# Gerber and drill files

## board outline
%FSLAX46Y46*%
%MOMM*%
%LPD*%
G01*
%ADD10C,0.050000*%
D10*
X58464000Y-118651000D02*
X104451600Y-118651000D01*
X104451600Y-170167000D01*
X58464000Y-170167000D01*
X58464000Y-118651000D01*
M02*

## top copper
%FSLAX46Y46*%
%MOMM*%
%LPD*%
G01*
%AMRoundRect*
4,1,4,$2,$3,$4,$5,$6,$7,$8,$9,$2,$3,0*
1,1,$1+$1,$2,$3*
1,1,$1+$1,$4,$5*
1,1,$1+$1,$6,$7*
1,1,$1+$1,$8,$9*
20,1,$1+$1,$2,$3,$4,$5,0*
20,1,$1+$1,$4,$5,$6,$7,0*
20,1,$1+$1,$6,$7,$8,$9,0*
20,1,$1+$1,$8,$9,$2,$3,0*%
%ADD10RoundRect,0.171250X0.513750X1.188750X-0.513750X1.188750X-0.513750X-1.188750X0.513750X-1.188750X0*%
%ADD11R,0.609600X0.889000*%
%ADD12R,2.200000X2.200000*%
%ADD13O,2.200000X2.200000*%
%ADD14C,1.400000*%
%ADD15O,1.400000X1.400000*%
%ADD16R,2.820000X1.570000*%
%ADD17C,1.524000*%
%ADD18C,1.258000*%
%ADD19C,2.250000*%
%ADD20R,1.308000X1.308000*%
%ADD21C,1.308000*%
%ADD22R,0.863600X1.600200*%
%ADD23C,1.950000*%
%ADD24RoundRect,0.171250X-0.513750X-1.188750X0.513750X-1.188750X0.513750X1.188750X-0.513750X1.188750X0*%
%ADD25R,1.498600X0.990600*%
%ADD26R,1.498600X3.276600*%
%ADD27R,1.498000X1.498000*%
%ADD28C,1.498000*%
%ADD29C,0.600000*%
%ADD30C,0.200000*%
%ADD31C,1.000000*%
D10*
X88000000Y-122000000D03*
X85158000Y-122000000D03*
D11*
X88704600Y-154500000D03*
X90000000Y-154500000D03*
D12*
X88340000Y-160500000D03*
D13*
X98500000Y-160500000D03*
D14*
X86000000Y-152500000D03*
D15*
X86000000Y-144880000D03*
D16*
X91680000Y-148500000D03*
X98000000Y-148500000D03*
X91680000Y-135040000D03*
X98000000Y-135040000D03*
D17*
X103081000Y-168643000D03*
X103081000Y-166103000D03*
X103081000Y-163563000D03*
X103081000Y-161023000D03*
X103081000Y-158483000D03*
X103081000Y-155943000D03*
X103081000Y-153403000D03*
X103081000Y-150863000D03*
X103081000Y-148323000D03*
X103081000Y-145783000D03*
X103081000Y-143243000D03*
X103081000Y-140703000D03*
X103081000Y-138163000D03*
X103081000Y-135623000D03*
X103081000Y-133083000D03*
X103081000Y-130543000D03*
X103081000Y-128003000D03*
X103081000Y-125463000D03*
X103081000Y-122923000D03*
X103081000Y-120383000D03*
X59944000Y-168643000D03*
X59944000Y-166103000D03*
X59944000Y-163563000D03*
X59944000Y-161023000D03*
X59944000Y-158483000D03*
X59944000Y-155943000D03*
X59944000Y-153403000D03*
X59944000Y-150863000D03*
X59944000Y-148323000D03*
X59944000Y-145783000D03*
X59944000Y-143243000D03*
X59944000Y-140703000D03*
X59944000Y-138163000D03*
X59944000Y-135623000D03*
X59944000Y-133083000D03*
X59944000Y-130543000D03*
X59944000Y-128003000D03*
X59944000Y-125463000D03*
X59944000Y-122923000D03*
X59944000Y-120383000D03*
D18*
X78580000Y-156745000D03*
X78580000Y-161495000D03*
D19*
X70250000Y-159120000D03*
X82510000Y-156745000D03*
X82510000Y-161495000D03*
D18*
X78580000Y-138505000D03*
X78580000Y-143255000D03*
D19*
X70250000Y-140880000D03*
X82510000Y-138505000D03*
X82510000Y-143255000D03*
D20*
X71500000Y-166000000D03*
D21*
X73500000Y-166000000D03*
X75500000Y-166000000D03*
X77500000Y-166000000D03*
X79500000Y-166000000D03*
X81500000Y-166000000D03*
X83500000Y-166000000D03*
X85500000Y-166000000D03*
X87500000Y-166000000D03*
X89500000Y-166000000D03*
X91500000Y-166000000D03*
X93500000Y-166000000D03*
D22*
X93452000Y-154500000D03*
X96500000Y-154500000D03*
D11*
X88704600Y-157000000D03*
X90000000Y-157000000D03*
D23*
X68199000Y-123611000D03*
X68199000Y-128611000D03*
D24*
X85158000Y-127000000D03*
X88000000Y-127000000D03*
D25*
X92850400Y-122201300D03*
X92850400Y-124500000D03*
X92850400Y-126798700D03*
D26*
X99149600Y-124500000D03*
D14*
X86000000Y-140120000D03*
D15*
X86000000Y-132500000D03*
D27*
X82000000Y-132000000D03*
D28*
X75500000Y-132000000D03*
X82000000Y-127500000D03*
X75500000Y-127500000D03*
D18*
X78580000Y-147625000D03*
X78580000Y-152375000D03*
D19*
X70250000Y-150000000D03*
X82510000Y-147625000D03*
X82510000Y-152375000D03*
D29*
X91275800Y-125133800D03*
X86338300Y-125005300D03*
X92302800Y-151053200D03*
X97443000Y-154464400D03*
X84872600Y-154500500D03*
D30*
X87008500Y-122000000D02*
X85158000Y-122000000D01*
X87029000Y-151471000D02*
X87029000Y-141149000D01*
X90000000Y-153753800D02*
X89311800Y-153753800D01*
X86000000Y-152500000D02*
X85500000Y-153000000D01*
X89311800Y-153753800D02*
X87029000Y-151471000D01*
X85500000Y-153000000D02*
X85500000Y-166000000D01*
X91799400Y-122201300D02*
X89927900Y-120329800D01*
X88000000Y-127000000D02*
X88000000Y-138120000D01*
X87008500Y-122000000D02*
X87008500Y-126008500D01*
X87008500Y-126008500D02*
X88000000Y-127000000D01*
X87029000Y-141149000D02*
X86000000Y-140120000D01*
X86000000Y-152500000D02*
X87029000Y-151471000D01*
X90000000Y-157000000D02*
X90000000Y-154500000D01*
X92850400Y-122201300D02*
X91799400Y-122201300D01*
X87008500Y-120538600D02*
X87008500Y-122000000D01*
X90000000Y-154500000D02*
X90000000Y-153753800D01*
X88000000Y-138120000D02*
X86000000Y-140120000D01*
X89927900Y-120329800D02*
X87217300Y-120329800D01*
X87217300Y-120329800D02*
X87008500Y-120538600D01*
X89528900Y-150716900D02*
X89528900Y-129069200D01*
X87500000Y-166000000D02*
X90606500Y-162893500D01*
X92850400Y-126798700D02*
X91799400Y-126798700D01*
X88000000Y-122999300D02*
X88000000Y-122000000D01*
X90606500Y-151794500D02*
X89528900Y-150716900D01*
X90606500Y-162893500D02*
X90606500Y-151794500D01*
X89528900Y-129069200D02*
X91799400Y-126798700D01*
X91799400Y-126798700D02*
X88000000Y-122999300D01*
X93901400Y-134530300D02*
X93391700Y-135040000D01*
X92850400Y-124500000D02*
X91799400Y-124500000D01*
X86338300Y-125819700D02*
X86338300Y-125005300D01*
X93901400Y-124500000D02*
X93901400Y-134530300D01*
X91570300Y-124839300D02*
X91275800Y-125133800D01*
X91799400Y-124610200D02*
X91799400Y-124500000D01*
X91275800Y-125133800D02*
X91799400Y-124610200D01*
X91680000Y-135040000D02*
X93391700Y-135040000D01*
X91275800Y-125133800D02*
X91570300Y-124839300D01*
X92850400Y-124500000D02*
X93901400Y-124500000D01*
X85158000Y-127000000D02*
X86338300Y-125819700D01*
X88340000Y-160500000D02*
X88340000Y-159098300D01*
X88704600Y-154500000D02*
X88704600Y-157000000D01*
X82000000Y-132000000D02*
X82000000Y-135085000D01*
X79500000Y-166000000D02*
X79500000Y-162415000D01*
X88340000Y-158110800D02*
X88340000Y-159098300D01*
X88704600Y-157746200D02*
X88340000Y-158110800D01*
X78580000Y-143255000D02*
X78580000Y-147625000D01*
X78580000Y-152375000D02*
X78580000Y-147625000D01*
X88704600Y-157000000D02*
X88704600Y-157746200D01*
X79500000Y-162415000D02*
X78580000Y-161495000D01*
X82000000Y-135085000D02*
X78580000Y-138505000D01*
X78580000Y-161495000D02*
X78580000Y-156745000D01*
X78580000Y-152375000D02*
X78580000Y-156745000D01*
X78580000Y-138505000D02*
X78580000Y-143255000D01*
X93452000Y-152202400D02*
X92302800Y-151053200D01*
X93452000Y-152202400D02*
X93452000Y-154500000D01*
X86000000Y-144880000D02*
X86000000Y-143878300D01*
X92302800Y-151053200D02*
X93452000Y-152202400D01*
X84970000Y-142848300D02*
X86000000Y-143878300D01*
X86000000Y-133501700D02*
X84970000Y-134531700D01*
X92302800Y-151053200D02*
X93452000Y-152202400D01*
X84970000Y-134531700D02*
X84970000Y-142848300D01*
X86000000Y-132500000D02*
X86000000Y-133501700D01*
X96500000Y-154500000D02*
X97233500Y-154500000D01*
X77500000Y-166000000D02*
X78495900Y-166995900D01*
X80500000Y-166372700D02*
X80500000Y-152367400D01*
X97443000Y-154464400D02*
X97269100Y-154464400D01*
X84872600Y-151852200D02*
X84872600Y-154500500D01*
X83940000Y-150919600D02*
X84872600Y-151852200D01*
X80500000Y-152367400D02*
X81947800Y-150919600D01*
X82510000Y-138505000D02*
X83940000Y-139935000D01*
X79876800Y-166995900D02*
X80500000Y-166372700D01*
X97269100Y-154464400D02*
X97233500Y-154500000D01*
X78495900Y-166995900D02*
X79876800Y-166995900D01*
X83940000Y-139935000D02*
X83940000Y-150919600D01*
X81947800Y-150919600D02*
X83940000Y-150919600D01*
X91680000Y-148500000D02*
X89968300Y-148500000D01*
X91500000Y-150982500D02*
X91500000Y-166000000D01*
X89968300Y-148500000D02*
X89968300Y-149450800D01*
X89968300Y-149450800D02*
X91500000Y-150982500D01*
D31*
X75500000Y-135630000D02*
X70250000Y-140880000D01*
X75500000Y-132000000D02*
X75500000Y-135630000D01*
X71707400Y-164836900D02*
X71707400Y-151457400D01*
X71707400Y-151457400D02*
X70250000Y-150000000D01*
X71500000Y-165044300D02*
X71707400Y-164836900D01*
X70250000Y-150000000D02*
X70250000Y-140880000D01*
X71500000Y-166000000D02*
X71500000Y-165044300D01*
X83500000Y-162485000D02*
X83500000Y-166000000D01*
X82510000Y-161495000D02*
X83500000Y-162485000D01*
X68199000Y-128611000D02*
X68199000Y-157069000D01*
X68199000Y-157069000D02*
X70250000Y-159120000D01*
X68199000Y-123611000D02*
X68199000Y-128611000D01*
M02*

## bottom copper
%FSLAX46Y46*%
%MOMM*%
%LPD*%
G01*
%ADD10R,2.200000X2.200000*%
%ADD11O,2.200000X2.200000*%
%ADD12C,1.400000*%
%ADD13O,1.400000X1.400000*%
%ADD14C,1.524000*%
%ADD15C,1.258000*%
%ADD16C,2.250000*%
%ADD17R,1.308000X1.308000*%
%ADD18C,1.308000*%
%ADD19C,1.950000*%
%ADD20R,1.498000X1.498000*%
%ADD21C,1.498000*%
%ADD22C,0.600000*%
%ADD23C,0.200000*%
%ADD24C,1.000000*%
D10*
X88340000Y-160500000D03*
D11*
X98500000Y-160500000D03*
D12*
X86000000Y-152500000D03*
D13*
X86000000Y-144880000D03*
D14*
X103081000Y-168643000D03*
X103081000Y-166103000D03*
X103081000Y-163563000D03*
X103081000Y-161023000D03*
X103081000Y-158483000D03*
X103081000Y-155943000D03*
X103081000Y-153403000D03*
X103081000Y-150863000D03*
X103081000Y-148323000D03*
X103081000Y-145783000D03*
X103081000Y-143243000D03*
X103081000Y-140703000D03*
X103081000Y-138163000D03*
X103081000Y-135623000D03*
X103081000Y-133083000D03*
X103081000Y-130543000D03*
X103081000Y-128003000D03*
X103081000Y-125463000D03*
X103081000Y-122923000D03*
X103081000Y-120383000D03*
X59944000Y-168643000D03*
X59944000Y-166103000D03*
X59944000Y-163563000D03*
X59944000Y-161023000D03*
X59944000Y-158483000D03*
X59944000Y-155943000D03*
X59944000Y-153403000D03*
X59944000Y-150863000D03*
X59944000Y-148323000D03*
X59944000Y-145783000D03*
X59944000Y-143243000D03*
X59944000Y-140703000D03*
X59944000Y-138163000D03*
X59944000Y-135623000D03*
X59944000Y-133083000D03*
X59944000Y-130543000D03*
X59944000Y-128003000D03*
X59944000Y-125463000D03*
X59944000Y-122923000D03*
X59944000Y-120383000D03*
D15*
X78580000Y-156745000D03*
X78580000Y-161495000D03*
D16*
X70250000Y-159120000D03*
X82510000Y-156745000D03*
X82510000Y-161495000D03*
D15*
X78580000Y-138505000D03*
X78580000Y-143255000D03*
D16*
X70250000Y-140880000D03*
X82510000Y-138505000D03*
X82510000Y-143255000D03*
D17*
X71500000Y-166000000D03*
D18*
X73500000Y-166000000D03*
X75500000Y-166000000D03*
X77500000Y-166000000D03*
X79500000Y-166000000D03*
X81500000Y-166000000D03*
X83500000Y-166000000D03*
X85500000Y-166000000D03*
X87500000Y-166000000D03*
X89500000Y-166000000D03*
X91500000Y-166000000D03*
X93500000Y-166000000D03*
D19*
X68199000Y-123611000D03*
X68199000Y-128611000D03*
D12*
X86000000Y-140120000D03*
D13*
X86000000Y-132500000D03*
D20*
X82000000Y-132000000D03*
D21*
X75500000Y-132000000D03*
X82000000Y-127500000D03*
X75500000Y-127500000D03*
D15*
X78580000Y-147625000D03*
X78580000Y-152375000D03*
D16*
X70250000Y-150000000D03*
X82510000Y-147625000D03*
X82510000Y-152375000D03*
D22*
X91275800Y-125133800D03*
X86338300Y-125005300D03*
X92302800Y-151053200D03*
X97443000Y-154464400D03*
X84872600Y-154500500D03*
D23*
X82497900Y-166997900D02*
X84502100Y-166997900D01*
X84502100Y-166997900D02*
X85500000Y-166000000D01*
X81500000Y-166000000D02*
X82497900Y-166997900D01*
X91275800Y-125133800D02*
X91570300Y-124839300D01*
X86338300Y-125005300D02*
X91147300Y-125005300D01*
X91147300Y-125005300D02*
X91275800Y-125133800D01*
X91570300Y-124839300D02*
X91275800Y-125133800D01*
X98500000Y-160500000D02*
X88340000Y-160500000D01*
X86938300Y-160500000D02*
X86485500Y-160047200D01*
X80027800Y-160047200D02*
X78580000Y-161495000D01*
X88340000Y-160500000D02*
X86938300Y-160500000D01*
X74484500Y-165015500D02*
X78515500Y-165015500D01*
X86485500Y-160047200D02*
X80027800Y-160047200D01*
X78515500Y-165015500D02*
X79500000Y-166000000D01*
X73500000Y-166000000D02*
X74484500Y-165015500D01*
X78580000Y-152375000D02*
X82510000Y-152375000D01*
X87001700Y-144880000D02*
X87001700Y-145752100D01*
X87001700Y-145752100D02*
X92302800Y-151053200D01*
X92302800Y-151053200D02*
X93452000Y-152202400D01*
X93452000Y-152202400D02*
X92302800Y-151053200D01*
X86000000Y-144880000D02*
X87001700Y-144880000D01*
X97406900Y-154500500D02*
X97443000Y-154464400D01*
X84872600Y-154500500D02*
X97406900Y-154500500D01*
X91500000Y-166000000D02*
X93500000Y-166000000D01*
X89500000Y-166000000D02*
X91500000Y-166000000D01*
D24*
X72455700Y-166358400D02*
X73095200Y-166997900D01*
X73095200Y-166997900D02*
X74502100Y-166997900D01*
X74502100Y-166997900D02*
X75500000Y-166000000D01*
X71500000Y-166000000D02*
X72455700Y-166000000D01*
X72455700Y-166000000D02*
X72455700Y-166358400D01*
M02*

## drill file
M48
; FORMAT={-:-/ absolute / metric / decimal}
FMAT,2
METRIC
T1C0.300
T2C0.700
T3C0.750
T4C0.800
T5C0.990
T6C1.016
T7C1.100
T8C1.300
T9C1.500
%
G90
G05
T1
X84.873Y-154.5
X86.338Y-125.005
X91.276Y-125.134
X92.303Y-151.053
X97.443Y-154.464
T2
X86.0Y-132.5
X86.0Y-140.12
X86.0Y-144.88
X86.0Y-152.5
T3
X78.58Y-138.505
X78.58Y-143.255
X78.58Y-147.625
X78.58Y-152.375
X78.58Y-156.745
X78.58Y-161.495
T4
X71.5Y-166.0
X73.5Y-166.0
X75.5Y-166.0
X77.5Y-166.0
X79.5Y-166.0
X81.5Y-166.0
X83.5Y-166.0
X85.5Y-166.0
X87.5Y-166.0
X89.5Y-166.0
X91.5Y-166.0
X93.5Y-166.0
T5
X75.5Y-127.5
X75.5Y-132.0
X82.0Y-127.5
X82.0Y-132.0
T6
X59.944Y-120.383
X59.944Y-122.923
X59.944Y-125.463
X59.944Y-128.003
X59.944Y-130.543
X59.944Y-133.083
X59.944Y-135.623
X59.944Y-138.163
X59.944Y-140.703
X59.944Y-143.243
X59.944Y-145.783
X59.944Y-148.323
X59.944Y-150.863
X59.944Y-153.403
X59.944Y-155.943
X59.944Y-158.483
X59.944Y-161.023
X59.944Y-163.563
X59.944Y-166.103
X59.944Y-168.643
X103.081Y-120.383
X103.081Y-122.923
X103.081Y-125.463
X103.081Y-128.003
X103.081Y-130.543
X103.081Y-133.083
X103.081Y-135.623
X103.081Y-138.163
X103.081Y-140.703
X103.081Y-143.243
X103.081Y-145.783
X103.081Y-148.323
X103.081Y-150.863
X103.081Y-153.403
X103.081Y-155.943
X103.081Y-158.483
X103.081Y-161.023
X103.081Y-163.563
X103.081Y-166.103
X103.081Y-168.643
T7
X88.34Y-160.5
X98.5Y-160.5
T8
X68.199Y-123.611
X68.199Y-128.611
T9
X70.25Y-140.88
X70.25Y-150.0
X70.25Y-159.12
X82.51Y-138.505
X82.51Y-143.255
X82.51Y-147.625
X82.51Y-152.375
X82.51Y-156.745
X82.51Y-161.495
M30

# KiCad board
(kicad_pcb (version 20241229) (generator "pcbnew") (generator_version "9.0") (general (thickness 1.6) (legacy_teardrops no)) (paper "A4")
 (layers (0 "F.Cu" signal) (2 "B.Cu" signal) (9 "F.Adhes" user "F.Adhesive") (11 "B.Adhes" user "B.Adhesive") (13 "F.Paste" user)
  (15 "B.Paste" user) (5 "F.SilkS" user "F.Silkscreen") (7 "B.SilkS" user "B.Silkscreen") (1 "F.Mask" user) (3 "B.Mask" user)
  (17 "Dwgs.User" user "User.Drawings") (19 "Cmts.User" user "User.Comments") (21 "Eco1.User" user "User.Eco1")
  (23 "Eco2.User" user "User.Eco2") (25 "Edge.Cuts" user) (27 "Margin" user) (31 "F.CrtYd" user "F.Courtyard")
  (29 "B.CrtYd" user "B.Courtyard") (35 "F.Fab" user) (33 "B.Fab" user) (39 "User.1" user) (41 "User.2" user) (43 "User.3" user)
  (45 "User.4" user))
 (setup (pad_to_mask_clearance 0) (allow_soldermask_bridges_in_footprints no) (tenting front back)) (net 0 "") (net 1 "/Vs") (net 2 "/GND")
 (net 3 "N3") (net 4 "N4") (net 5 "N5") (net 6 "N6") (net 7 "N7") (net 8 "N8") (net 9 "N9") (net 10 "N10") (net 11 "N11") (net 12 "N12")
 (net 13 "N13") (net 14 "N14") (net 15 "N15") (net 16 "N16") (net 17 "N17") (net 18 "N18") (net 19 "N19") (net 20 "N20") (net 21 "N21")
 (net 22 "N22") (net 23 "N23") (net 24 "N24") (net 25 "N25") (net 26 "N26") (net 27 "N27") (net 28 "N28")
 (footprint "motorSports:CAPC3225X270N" (layer "F.Cu") (at 86.579 122 180)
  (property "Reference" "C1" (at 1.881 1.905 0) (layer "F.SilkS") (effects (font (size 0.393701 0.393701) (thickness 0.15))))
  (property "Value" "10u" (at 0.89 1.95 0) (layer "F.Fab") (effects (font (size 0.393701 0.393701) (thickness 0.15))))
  (pad "1" smd roundrect (at -1.421 0 180) (size 1.37 2.72) (layers "F.Cu" "F.Mask" "F.Paste") (roundrect_rratio 0.125) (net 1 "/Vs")
   (solder_mask_margin 0.102))
  (pad "2" smd roundrect (at 1.421 0 180) (size 1.37 2.72) (layers "F.Cu" "F.Mask" "F.Paste") (roundrect_rratio 0.125) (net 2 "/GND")
   (solder_mask_margin 0.102)))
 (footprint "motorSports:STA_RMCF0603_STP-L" (layer "F.Cu") (at 89.3523 154.5)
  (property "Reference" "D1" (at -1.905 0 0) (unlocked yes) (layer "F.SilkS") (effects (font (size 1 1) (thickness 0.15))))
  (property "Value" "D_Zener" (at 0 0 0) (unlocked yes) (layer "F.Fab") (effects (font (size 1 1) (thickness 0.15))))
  (pad "1" smd rect (at -0.6477 0) (size 0.6096 0.889) (layers "F.Cu" "F.Mask" "F.Paste") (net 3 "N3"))
  (pad "2" smd rect (at 0.6477 0) (size 0.6096 0.889) (layers "F.Cu" "F.Mask" "F.Paste") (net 2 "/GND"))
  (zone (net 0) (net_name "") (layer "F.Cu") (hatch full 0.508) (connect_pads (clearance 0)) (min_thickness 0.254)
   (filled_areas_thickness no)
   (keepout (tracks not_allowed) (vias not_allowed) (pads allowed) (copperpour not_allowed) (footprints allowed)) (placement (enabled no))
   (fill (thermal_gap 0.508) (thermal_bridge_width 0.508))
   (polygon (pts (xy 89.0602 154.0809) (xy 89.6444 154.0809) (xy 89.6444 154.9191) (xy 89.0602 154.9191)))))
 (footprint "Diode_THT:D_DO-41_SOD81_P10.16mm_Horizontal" (layer "F.Cu") (at 88.34 160.5)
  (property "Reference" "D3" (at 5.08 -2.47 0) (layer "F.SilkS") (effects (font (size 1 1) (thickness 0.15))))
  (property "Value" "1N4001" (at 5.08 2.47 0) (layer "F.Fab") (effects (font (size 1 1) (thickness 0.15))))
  (pad "1" thru_hole rect (at 0 0) (size 2.2 2.2) (drill 1.1) (layers "*.Cu" "*.Mask") (remove_unused_layers no) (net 3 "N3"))
  (pad "2" thru_hole oval (at 10.16 0) (size 2.2 2.2) (drill 1.1) (layers "*.Cu" "*.Mask") (remove_unused_layers no) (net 3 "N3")))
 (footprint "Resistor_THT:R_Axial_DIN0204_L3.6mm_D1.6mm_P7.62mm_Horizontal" (layer "F.Cu") (at 86 152.5 90)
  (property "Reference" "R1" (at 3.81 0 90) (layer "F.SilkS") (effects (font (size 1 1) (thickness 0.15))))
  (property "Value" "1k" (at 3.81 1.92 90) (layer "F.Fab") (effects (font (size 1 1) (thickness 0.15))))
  (pad "1" thru_hole circle (at 0 0 90) (size 1.4 1.4) (drill 0.7) (layers "*.Cu" "*.Mask") (remove_unused_layers no) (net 2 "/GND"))
  (pad "2" thru_hole oval (at 7.62 0 90) (size 1.4 1.4) (drill 0.7) (layers "*.Cu" "*.Mask") (remove_unused_layers no) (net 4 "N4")))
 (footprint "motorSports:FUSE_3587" (layer "F.Cu") (at 94.84 141.77 90)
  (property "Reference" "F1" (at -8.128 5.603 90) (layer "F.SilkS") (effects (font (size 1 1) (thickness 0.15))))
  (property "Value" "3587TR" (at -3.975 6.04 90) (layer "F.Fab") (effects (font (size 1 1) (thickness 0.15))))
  (pad "1_1" smd rect (at -6.73 -3.16 90) (size 1.57 2.82) (layers "F.Cu" "F.Mask" "F.Paste") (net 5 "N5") (solder_mask_margin 0.102))
  (pad "1_2" smd rect (at -6.73 3.16 90) (size 1.57 2.82) (layers "F.Cu" "F.Mask" "F.Paste") (solder_mask_margin 0.102))
  (pad "2_1" smd rect (at 6.73 -3.16 90) (size 1.57 2.82) (layers "F.Cu" "F.Mask" "F.Paste") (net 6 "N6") (solder_mask_margin 0.102))
  (pad "2_2" smd rect (at 6.73 3.16 90) (size 1.57 2.82) (layers "F.Cu" "F.Mask" "F.Paste") (solder_mask_margin 0.102)))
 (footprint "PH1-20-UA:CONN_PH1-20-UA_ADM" (layer "F.Cu") (at 103.081 168.643 90)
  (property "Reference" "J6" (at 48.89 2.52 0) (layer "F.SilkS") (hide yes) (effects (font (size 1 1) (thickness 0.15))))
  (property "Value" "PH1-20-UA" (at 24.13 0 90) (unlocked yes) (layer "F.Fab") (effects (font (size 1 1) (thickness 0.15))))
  (pad "1" thru_hole circle (at 0 0 90) (size 1.524 1.524) (drill 1.016) (layers "*.Cu" "*.Mask") (remove_unused_layers no))
  (pad "2" thru_hole circle (at 2.54 0 90) (size 1.524 1.524) (drill 1.016) (layers "*.Cu" "*.Mask") (remove_unused_layers no))
  (pad "3" thru_hole circle (at 5.08 0 90) (size 1.524 1.524) (drill 1.016) (layers "*.Cu" "*.Mask") (remove_unused_layers no))
  (pad "4" thru_hole circle (at 7.62 0 90) (size 1.524 1.524) (drill 1.016) (layers "*.Cu" "*.Mask") (remove_unused_layers no))
  (pad "5" thru_hole circle (at 10.16 0 90) (size 1.524 1.524) (drill 1.016) (layers "*.Cu" "*.Mask") (remove_unused_layers no))
  (pad "6" thru_hole circle (at 12.7 0 90) (size 1.524 1.524) (drill 1.016) (layers "*.Cu" "*.Mask") (remove_unused_layers no))
  (pad "7" thru_hole circle (at 15.24 0 90) (size 1.524 1.524) (drill 1.016) (layers "*.Cu" "*.Mask") (remove_unused_layers no))
  (pad "8" thru_hole circle (at 17.78 0 90) (size 1.524 1.524) (drill 1.016) (layers "*.Cu" "*.Mask") (remove_unused_layers no))
  (pad "9" thru_hole circle (at 20.32 0 90) (size 1.524 1.524) (drill 1.016) (layers "*.Cu" "*.Mask") (remove_unused_layers no))
  (pad "10" thru_hole circle (at 22.86 0 90) (size 1.524 1.524) (drill 1.016) (layers "*.Cu" "*.Mask") (remove_unused_layers no))
  (pad "11" thru_hole circle (at 25.4 0 90) (size 1.524 1.524) (drill 1.016) (layers "*.Cu" "*.Mask") (remove_unused_layers no))
  (pad "12" thru_hole circle (at 27.94 0 90) (size 1.524 1.524) (drill 1.016) (layers "*.Cu" "*.Mask") (remove_unused_layers no))
  (pad "13" thru_hole circle (at 30.48 0 90) (size 1.524 1.524) (drill 1.016) (layers "*.Cu" "*.Mask") (remove_unused_layers no))
  (pad "14" thru_hole circle (at 33.02 0 90) (size 1.524 1.524) (drill 1.016) (layers "*.Cu" "*.Mask") (remove_unused_layers no))
  (pad "15" thru_hole circle (at 35.56 0 90) (size 1.524 1.524) (drill 1.016) (layers "*.Cu" "*.Mask") (remove_unused_layers no))
  (pad "16" thru_hole circle (at 38.1 0 90) (size 1.524 1.524) (drill 1.016) (layers "*.Cu" "*.Mask") (remove_unused_layers no))
  (pad "17" thru_hole circle (at 40.64 0 90) (size 1.524 1.524) (drill 1.016) (layers "*.Cu" "*.Mask") (remove_unused_layers no))
  (pad "18" thru_hole circle (at 43.18 0 90) (size 1.524 1.524) (drill 1.016) (layers "*.Cu" "*.Mask") (remove_unused_layers no))
  (pad "19" thru_hole circle (at 45.72 0 90) (size 1.524 1.524) (drill 1.016) (layers "*.Cu" "*.Mask") (remove_unused_layers no))
  (pad "20" thru_hole circle (at 48.26 0 90) (size 1.524 1.524) (drill 1.016) (layers "*.Cu" "*.Mask") (remove_unused_layers no)))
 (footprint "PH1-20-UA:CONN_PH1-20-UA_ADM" (layer "F.Cu") (at 59.944 168.643 90)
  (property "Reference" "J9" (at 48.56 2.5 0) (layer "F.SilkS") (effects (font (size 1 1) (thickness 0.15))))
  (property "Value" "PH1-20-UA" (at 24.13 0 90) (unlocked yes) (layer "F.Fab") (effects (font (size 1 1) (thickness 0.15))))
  (pad "1" thru_hole circle (at 0 0 90) (size 1.524 1.524) (drill 1.016) (layers "*.Cu" "*.Mask") (remove_unused_layers no))
  (pad "2" thru_hole circle (at 2.54 0 90) (size 1.524 1.524) (drill 1.016) (layers "*.Cu" "*.Mask") (remove_unused_layers no))
  (pad "3" thru_hole circle (at 5.08 0 90) (size 1.524 1.524) (drill 1.016) (layers "*.Cu" "*.Mask") (remove_unused_layers no) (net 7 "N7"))
  (pad "4" thru_hole circle (at 7.62 0 90) (size 1.524 1.524) (drill 1.016) (layers "*.Cu" "*.Mask") (remove_unused_layers no))
  (pad "5" thru_hole circle (at 10.16 0 90) (size 1.524 1.524) (drill 1.016) (layers "*.Cu" "*.Mask") (remove_unused_layers no))
  (pad "6" thru_hole circle (at 12.7 0 90) (size 1.524 1.524) (drill 1.016) (layers "*.Cu" "*.Mask") (remove_unused_layers no))
  (pad "7" thru_hole circle (at 15.24 0 90) (size 1.524 1.524) (drill 1.016) (layers "*.Cu" "*.Mask") (remove_unused_layers no) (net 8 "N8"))
  (pad "8" thru_hole circle (at 17.78 0 90) (size 1.524 1.524) (drill 1.016) (layers "*.Cu" "*.Mask") (remove_unused_layers no) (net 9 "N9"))
  (pad "9" thru_hole circle (at 20.32 0 90) (size 1.524 1.524) (drill 1.016) (layers "*.Cu" "*.Mask") (remove_unused_layers no)
   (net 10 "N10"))
  (pad "10" thru_hole circle (at 22.86 0 90) (size 1.524 1.524) (drill 1.016) (layers "*.Cu" "*.Mask") (remove_unused_layers no)
   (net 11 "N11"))
  (pad "11" thru_hole circle (at 25.4 0 90) (size 1.524 1.524) (drill 1.016) (layers "*.Cu" "*.Mask") (remove_unused_layers no)
   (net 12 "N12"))
  (pad "12" thru_hole circle (at 27.94 0 90) (size 1.524 1.524) (drill 1.016) (layers "*.Cu" "*.Mask") (remove_unused_layers no)
   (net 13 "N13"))
  (pad "13" thru_hole circle (at 30.48 0 90) (size 1.524 1.524) (drill 1.016) (layers "*.Cu" "*.Mask") (remove_unused_layers no)
   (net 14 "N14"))
  (pad "14" thru_hole circle (at 33.02 0 90) (size 1.524 1.524) (drill 1.016) (layers "*.Cu" "*.Mask") (remove_unused_layers no)
   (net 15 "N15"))
  (pad "15" thru_hole circle (at 35.56 0 90) (size 1.524 1.524) (drill 1.016) (layers "*.Cu" "*.Mask") (remove_unused_layers no)
   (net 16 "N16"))
  (pad "16" thru_hole circle (at 38.1 0 90) (size 1.524 1.524) (drill 1.016) (layers "*.Cu" "*.Mask") (remove_unused_layers no)
   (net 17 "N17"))
  (pad "17" thru_hole circle (at 40.64 0 90) (size 1.524 1.524) (drill 1.016) (layers "*.Cu" "*.Mask") (remove_unused_layers no)
   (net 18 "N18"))
  (pad "18" thru_hole circle (at 43.18 0 90) (size 1.524 1.524) (drill 1.016) (layers "*.Cu" "*.Mask") (remove_unused_layers no)
   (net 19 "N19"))
  (pad "19" thru_hole circle (at 45.72 0 90) (size 1.524 1.524) (drill 1.016) (layers "*.Cu" "*.Mask") (remove_unused_layers no)
   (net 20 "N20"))
  (pad "20" thru_hole circle (at 48.26 0 90) (size 1.524 1.524) (drill 1.016) (layers "*.Cu" "*.Mask") (remove_unused_layers no)
   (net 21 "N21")))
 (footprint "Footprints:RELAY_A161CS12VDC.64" (layer "F.Cu") (at 76.5 159.12)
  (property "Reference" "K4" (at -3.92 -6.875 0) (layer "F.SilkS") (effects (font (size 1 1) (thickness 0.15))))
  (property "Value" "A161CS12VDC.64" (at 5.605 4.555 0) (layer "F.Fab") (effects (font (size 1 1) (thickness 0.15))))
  (pad "A1" thru_hole circle (at 2.08 -2.375) (size 1.258 1.258) (drill 0.75) (layers "*.Cu" "*.Mask") (remove_unused_layers no)
   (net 3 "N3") (solder_mask_margin 0.102))
  (pad "A2" thru_hole circle (at 2.08 2.375) (size 1.258 1.258) (drill 0.75) (layers "*.Cu" "*.Mask") (remove_unused_layers no) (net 3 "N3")
   (solder_mask_margin 0.102))
  (pad "COM" thru_hole circle (at -6.25 0) (size 2.25 2.25) (drill 1.5) (layers "*.Cu" "*.Mask") (remove_unused_layers no) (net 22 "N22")
   (solder_mask_margin 0.102))
  (pad "NC" thru_hole circle (at 6.01 -2.375) (size 2.25 2.25) (drill 1.5) (layers "*.Cu" "*.Mask") (remove_unused_layers no) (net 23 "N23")
   (solder_mask_margin 0.102))
  (pad "NO" thru_hole circle (at 6.01 2.375) (size 2.25 2.25) (drill 1.5) (layers "*.Cu" "*.Mask") (remove_unused_layers no) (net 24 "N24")
   (solder_mask_margin 0.102)))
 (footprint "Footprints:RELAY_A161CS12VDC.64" (layer "F.Cu") (at 76.5 140.88)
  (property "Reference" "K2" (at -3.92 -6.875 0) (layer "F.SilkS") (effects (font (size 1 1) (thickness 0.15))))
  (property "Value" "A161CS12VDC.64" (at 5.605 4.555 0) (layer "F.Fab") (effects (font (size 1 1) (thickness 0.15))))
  (pad "A1" thru_hole circle (at 2.08 -2.375) (size 1.258 1.258) (drill 0.75) (layers "*.Cu" "*.Mask") (remove_unused_layers no)
   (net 3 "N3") (solder_mask_margin 0.102))
  (pad "A2" thru_hole circle (at 2.08 2.375) (size 1.258 1.258) (drill 0.75) (layers "*.Cu" "*.Mask") (remove_unused_layers no) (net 3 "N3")
   (solder_mask_margin 0.102))
  (pad "COM" thru_hole circle (at -6.25 0) (size 2.25 2.25) (drill 1.5) (layers "*.Cu" "*.Mask") (remove_unused_layers no) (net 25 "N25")
   (solder_mask_margin 0.102))
  (pad "NC" thru_hole circle (at 6.01 -2.375) (size 2.25 2.25) (drill 1.5) (layers "*.Cu" "*.Mask") (remove_unused_layers no) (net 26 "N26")
   (solder_mask_margin 0.102))
  (pad "NO" thru_hole circle (at 6.01 2.375) (size 2.25 2.25) (drill 1.5) (layers "*.Cu" "*.Mask") (remove_unused_layers no) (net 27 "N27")
   (solder_mask_margin 0.102)))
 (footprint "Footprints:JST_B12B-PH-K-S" (layer "F.Cu") (at 82.5 166.55 180)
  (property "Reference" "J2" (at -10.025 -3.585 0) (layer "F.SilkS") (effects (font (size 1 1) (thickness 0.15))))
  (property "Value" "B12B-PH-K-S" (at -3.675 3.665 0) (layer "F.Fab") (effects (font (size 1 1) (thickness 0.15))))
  (pad "1" thru_hole rect (at 11 0.55 180) (size 1.308 1.308) (drill 0.8) (layers "*.Cu" "*.Mask") (remove_unused_layers no) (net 25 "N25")
   (solder_mask_margin 0.102))
  (pad "2" thru_hole circle (at 9 0.55 180) (size 1.308 1.308) (drill 0.8) (layers "*.Cu" "*.Mask") (remove_unused_layers no) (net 3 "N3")
   (solder_mask_margin 0.102))
  (pad "3" thru_hole circle (at 7 0.55 180) (size 1.308 1.308) (drill 0.8) (layers "*.Cu" "*.Mask") (remove_unused_layers no) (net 25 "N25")
   (solder_mask_margin 0.102))
  (pad "4" thru_hole circle (at 5 0.55 180) (size 1.308 1.308) (drill 0.8) (layers "*.Cu" "*.Mask") (remove_unused_layers no) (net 26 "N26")
   (solder_mask_margin 0.102))
  (pad "5" thru_hole circle (at 3 0.55 180) (size 1.308 1.308) (drill 0.8) (layers "*.Cu" "*.Mask") (remove_unused_layers no) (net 3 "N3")
   (solder_mask_margin 0.102))
  (pad "6" thru_hole circle (at 1 0.55 180) (size 1.308 1.308) (drill 0.8) (layers "*.Cu" "*.Mask") (remove_unused_layers no) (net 2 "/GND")
   (solder_mask_margin 0.102))
  (pad "7" thru_hole circle (at -1 0.55 180) (size 1.308 1.308) (drill 0.8) (layers "*.Cu" "*.Mask") (remove_unused_layers no)
   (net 24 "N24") (solder_mask_margin 0.102))
  (pad "8" thru_hole circle (at -3 0.55 180) (size 1.308 1.308) (drill 0.8) (layers "*.Cu" "*.Mask") (remove_unused_layers no)
   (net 2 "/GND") (solder_mask_margin 0.102))
  (pad "9" thru_hole circle (at -5 0.55 180) (size 1.308 1.308) (drill 0.8) (layers "*.Cu" "*.Mask") (remove_unused_layers no) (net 1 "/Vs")
   (solder_mask_margin 0.102))
  (pad "10" thru_hole circle (at -7 0.55 180) (size 1.308 1.308) (drill 0.8) (layers "*.Cu" "*.Mask") (remove_unused_layers no) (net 5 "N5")
   (solder_mask_margin 0.102))
  (pad "11" thru_hole circle (at -9 0.55 180) (size 1.308 1.308) (drill 0.8) (layers "*.Cu" "*.Mask") (remove_unused_layers no) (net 5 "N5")
   (solder_mask_margin 0.102))
  (pad "12" thru_hole circle (at -11 0.55 180) (size 1.308 1.308) (drill 0.8) (layers "*.Cu" "*.Mask") (remove_unused_layers no)
   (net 5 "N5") (solder_mask_margin 0.102)))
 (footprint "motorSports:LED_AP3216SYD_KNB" (layer "F.Cu") (at 94.976 154.5)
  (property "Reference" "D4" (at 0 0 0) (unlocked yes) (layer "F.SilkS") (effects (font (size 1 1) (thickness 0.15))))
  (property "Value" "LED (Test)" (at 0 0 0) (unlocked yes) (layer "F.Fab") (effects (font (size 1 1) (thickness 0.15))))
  (pad "1" smd rect (at -1.524 0) (size 0.8636 1.6002) (layers "F.Cu" "F.Mask" "F.Paste") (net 4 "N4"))
  (pad "2" smd rect (at 1.524 0) (size 0.8636 1.6002) (layers "F.Cu" "F.Mask" "F.Paste") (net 26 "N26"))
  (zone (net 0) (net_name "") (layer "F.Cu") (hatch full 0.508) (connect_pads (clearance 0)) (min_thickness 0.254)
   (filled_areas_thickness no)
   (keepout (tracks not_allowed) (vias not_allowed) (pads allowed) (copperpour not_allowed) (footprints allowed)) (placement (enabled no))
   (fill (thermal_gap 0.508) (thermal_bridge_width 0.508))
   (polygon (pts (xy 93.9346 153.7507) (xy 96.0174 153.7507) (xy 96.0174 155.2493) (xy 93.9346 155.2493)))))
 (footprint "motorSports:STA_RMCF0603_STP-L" (layer "F.Cu") (at 89.3523 157)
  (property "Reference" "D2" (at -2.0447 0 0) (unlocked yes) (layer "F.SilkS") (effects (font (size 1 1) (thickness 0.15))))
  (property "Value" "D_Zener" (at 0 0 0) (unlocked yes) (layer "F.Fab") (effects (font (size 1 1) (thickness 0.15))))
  (pad "1" smd rect (at -0.6477 0) (size 0.6096 0.889) (layers "F.Cu" "F.Mask" "F.Paste") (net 3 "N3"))
  (pad "2" smd rect (at 0.6477 0) (size 0.6096 0.889) (layers "F.Cu" "F.Mask" "F.Paste") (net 2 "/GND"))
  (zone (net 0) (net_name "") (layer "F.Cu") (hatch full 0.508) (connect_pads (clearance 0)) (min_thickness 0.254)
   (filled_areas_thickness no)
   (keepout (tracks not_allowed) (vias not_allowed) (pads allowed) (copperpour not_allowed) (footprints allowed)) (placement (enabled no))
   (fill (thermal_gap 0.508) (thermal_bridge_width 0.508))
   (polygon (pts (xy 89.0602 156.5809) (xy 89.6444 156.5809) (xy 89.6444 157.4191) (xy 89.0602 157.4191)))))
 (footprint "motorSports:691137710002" (layer "F.Cu") (at 68.199 126.111 -90)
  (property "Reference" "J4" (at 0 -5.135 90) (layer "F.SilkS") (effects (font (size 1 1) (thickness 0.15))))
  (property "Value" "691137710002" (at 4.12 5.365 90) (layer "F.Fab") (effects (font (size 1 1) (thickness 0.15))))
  (pad "1" thru_hole circle (at -2.5 0 270) (size 1.95 1.95) (drill 1.3) (layers "*.Cu" "*.Mask") (remove_unused_layers no) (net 22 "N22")
   (solder_mask_margin 0.102))
  (pad "2" thru_hole circle (at 2.5 0 270) (size 1.95 1.95) (drill 1.3) (layers "*.Cu" "*.Mask") (remove_unused_layers no) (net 22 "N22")
   (solder_mask_margin 0.102)))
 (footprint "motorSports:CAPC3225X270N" (layer "F.Cu") (at 86.579 127)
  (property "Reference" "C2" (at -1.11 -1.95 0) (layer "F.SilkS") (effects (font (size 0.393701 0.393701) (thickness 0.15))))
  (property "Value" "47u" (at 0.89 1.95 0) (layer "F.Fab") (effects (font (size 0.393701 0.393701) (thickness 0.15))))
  (pad "1" smd roundrect (at -1.421 0) (size 1.37 2.72) (layers "F.Cu" "F.Mask" "F.Paste") (roundrect_rratio 0.125) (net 6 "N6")
   (solder_mask_margin 0.102))
  (pad "2" smd roundrect (at 1.421 0) (size 1.37 2.72) (layers "F.Cu" "F.Mask" "F.Paste") (roundrect_rratio 0.125) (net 2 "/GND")
   (solder_mask_margin 0.102)))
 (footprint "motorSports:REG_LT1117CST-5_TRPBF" (layer "F.Cu") (at 96 124.5)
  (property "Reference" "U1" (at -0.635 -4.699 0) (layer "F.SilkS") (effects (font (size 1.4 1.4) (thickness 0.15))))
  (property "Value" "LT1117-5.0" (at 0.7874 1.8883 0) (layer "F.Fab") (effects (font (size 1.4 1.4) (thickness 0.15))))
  (pad "1" smd rect (at -3.1496 -2.2987) (size 1.4986 0.9906) (layers "F.Cu" "F.Mask" "F.Paste") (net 2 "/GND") (solder_mask_margin 0.102))
  (pad "2" smd rect (at -3.1496 0) (size 1.4986 0.9906) (layers "F.Cu" "F.Mask" "F.Paste") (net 6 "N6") (solder_mask_margin 0.102))
  (pad "3" smd rect (at -3.1496 2.2987) (size 1.4986 0.9906) (layers "F.Cu" "F.Mask" "F.Paste") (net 1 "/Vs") (solder_mask_margin 0.102))
  (pad "4" smd rect (at 3.1496 0) (size 1.4986 3.2766) (layers "F.Cu" "F.Mask" "F.Paste") (solder_mask_margin 0.102)))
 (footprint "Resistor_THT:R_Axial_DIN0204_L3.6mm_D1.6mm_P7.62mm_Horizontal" (layer "F.Cu") (at 86 140.12 90)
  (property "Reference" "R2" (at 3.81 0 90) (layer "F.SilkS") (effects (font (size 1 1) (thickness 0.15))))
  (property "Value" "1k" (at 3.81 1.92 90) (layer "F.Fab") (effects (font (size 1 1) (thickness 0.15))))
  (pad "1" thru_hole circle (at 0 0 90) (size 1.4 1.4) (drill 0.7) (layers "*.Cu" "*.Mask") (remove_unused_layers no) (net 2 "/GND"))
  (pad "2" thru_hole oval (at 7.62 0 90) (size 1.4 1.4) (drill 0.7) (layers "*.Cu" "*.Mask") (remove_unused_layers no) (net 4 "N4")))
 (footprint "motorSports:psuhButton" (layer "F.Cu") (at 78.75 129.75 180)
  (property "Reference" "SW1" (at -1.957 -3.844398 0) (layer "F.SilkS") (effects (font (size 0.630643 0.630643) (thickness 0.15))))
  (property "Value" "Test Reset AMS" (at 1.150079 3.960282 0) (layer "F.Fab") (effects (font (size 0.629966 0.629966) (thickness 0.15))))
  (pad "1" thru_hole rect (at -3.25 -2.25 180) (size 1.498 1.498) (drill 0.99) (layers "*.Cu" "*.Mask") (remove_unused_layers no)
   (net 3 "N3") (solder_mask_margin 0.102))
  (pad "2" thru_hole circle (at 3.25 -2.25 180) (size 1.498 1.498) (drill 0.99) (layers "*.Cu" "*.Mask") (remove_unused_layers no)
   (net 25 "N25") (solder_mask_margin 0.102))
  (pad "3" thru_hole circle (at -3.25 2.25 180) (size 1.498 1.498) (drill 0.99) (layers "*.Cu" "*.Mask") (remove_unused_layers no)
   (solder_mask_margin 0.102))
  (pad "4" thru_hole circle (at 3.25 2.25 180) (size 1.498 1.498) (drill 0.99) (layers "*.Cu" "*.Mask") (remove_unused_layers no)
   (solder_mask_margin 0.102)))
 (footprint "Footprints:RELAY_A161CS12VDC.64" (layer "F.Cu") (at 76.5 150)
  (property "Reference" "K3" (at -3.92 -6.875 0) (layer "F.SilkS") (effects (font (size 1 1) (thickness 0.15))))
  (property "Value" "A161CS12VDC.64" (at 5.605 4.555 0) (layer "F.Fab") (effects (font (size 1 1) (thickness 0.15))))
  (pad "A1" thru_hole circle (at 2.08 -2.375) (size 1.258 1.258) (drill 0.75) (layers "*.Cu" "*.Mask") (remove_unused_layers no)
   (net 3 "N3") (solder_mask_margin 0.102))
  (pad "A2" thru_hole circle (at 2.08 2.375) (size 1.258 1.258) (drill 0.75) (layers "*.Cu" "*.Mask") (remove_unused_layers no) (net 3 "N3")
   (solder_mask_margin 0.102))
  (pad "COM" thru_hole circle (at -6.25 0) (size 2.25 2.25) (drill 1.5) (layers "*.Cu" "*.Mask") (remove_unused_layers no) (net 25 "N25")
   (solder_mask_margin 0.102))
  (pad "NC" thru_hole circle (at 6.01 -2.375) (size 2.25 2.25) (drill 1.5) (layers "*.Cu" "*.Mask") (remove_unused_layers no) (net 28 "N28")
   (solder_mask_margin 0.102))
  (pad "NO" thru_hole circle (at 6.01 2.375) (size 2.25 2.25) (drill 1.5) (layers "*.Cu" "*.Mask") (remove_unused_layers no) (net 3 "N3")
   (solder_mask_margin 0.102)))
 (gr_rect (start 58.464 118.651) (end 104.4516 170.167) (stroke (width 0.05) (type default)) (fill no) (layer "Edge.Cuts"))
 (segment (start 87.0085 122) (end 85.158 122) (width 0.2) (layer "F.Cu") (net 2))
 (segment (start 87.029 151.471) (end 87.029 141.149) (width 0.2) (layer "F.Cu") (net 2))
 (segment (start 90 153.7538) (end 89.3118 153.7538) (width 0.2) (layer "F.Cu") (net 2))
 (segment (start 86 152.5) (end 85.5 153) (width 0.2) (layer "F.Cu") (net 2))
 (segment (start 89.3118 153.7538) (end 87.029 151.471) (width 0.2) (layer "F.Cu") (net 2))
 (segment (start 85.5 153) (end 85.5 166) (width 0.2) (layer "F.Cu") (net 2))
 (segment (start 91.7994 122.2013) (end 89.9279 120.3298) (width 0.2) (layer "F.Cu") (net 2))
 (segment (start 88 127) (end 88 138.12) (width 0.2) (layer "F.Cu") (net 2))
 (segment (start 87.0085 122) (end 87.0085 126.0085) (width 0.2) (layer "F.Cu") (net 2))
 (segment (start 87.0085 126.0085) (end 88 127) (width 0.2) (layer "F.Cu") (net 2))
 (segment (start 87.029 141.149) (end 86 140.12) (width 0.2) (layer "F.Cu") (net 2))
 (segment (start 86 152.5) (end 87.029 151.471) (width 0.2) (layer "F.Cu") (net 2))
 (segment (start 90 157) (end 90 154.5) (width 0.2) (layer "F.Cu") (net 2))
 (segment (start 92.8504 122.2013) (end 91.7994 122.2013) (width 0.2) (layer "F.Cu") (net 2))
 (segment (start 87.0085 120.5386) (end 87.0085 122) (width 0.2) (layer "F.Cu") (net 2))
 (segment (start 90 154.5) (end 90 153.7538) (width 0.2) (layer "F.Cu") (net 2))
 (segment (start 88 138.12) (end 86 140.12) (width 0.2) (layer "F.Cu") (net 2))
 (segment (start 89.9279 120.3298) (end 87.2173 120.3298) (width 0.2) (layer "F.Cu") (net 2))
 (segment (start 87.2173 120.3298) (end 87.0085 120.5386) (width 0.2) (layer "F.Cu") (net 2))
 (segment (start 82.4979 166.9979) (end 84.5021 166.9979) (width 0.2) (layer "B.Cu") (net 2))
 (segment (start 84.5021 166.9979) (end 85.5 166) (width 0.2) (layer "B.Cu") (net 2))
 (segment (start 81.5 166) (end 82.4979 166.9979) (width 0.2) (layer "B.Cu") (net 2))
 (segment (start 89.5289 150.7169) (end 89.5289 129.0692) (width 0.2) (layer "F.Cu") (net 1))
 (segment (start 87.5 166) (end 90.6065 162.8935) (width 0.2) (layer "F.Cu") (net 1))
 (segment (start 92.8504 126.7987) (end 91.7994 126.7987) (width 0.2) (layer "F.Cu") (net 1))
 (segment (start 88 122.9993) (end 88 122) (width 0.2) (layer "F.Cu") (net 1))
 (segment (start 90.6065 151.7945) (end 89.5289 150.7169) (width 0.2) (layer "F.Cu") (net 1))
 (segment (start 90.6065 162.8935) (end 90.6065 151.7945) (width 0.2) (layer "F.Cu") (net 1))
 (segment (start 89.5289 129.0692) (end 91.7994 126.7987) (width 0.2) (layer "F.Cu") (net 1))
 (segment (start 91.7994 126.7987) (end 88 122.9993) (width 0.2) (layer "F.Cu") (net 1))
 (segment (start 93.9014 134.5303) (end 93.3917 135.04) (width 0.2) (layer "F.Cu") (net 6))
 (segment (start 92.8504 124.5) (end 91.7994 124.5) (width 0.2) (layer "F.Cu") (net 6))
 (segment (start 86.3383 125.8197) (end 86.3383 125.0053) (width 0.2) (layer "F.Cu") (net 6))
 (segment (start 93.9014 124.5) (end 93.9014 134.5303) (width 0.2) (layer "F.Cu") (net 6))
 (segment (start 91.5703 124.8393) (end 91.2758 125.1338) (width 0.2) (layer "F.Cu") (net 6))
 (segment (start 91.7994 124.6102) (end 91.7994 124.5) (width 0.2) (layer "F.Cu") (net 6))
 (segment (start 91.2758 125.1338) (end 91.7994 124.6102) (width 0.2) (layer "F.Cu") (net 6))
 (segment (start 91.68 135.04) (end 93.3917 135.04) (width 0.2) (layer "F.Cu") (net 6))
 (segment (start 91.2758 125.1338) (end 91.5703 124.8393) (width 0.2) (layer "F.Cu") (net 6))
 (segment (start 92.8504 124.5) (end 93.9014 124.5) (width 0.2) (layer "F.Cu") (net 6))
 (segment (start 85.158 127) (end 86.3383 125.8197) (width 0.2) (layer "F.Cu") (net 6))
 (via (at 91.2758 125.1338) (size 0.6) (drill 0.3) (layers "F.Cu" "B.Cu") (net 6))
 (via (at 86.3383 125.0053) (size 0.6) (drill 0.3) (layers "F.Cu" "B.Cu") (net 6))
 (segment (start 91.2758 125.1338) (end 91.5703 124.8393) (width 0.2) (layer "B.Cu") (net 6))
 (segment (start 86.3383 125.0053) (end 91.1473 125.0053) (width 0.2) (layer "B.Cu") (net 6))
 (segment (start 91.1473 125.0053) (end 91.2758 125.1338) (width 0.2) (layer "B.Cu") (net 6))
 (segment (start 91.5703 124.8393) (end 91.2758 125.1338) (width 0.2) (layer "B.Cu") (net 6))
 (segment (start 88.34 160.5) (end 88.34 159.0983) (width 0.2) (layer "F.Cu") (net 3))
 (segment (start 88.7046 154.5) (end 88.7046 157) (width 0.2) (layer "F.Cu") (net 3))
 (segment (start 82 132) (end 82 135.085) (width 0.2) (layer "F.Cu") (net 3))
 (segment (start 79.5 166) (end 79.5 162.415) (width 0.2) (layer "F.Cu") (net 3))
 (segment (start 88.34 158.1108) (end 88.34 159.0983) (width 0.2) (layer "F.Cu") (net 3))
 (segment (start 88.7046 157.7462) (end 88.34 158.1108) (width 0.2) (layer "F.Cu") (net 3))
 (segment (start 78.58 143.255) (end 78.58 147.625) (width 0.2) (layer "F.Cu") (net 3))
 (segment (start 78.58 152.375) (end 78.58 147.625) (width 0.2) (layer "F.Cu") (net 3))
 (segment (start 88.7046 157) (end 88.7046 157.7462) (width 0.2) (layer "F.Cu") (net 3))
 (segment (start 79.5 162.415) (end 78.58 161.495) (width 0.2) (layer "F.Cu") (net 3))
 (segment (start 82 135.085) (end 78.58 138.505) (width 0.2) (layer "F.Cu") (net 3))
 (segment (start 78.58 161.495) (end 78.58 156.745) (width 0.2) (layer "F.Cu") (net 3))
 (segment (start 78.58 152.375) (end 78.58 156.745) (width 0.2) (layer "F.Cu") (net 3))
 (segment (start 78.58 138.505) (end 78.58 143.255) (width 0.2) (layer "F.Cu") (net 3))
 (segment (start 98.5 160.5) (end 88.34 160.5) (width 0.2) (layer "B.Cu") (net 3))
 (segment (start 86.9383 160.5) (end 86.4855 160.0472) (width 0.2) (layer "B.Cu") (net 3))
 (segment (start 80.0278 160.0472) (end 78.58 161.495) (width 0.2) (layer "B.Cu") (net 3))
 (segment (start 88.34 160.5) (end 86.9383 160.5) (width 0.2) (layer "B.Cu") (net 3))
 (segment (start 74.4845 165.0155) (end 78.5155 165.0155) (width 0.2) (layer "B.Cu") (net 3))
 (segment (start 86.4855 160.0472) (end 80.0278 160.0472) (width 0.2) (layer "B.Cu") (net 3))
 (segment (start 78.5155 165.0155) (end 79.5 166) (width 0.2) (layer "B.Cu") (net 3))
 (segment (start 73.5 166) (end 74.4845 165.0155) (width 0.2) (layer "B.Cu") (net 3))
 (segment (start 78.58 152.375) (end 82.51 152.375) (width 0.2) (layer "B.Cu") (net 3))
 (segment (start 93.452 152.2024) (end 92.3028 151.0532) (width 0.2) (layer "F.Cu") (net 4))
 (segment (start 93.452 152.2024) (end 93.452 154.5) (width 0.2) (layer "F.Cu") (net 4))
 (segment (start 86 144.88) (end 86 143.8783) (width 0.2) (layer "F.Cu") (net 4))
 (segment (start 92.3028 151.0532) (end 93.452 152.2024) (width 0.2) (layer "F.Cu") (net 4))
 (segment (start 84.97 142.8483) (end 86 143.8783) (width 0.2) (layer "F.Cu") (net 4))
 (segment (start 86 133.5017) (end 84.97 134.5317) (width 0.2) (layer "F.Cu") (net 4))
 (segment (start 92.3028 151.0532) (end 93.452 152.2024) (width 0.2) (layer "F.Cu") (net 4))
 (segment (start 84.97 134.5317) (end 84.97 142.8483) (width 0.2) (layer "F.Cu") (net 4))
 (segment (start 86 132.5) (end 86 133.5017) (width 0.2) (layer "F.Cu") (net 4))
 (via (at 92.3028 151.0532) (size 0.6) (drill 0.3) (layers "F.Cu" "B.Cu") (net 4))
 (segment (start 87.0017 144.88) (end 87.0017 145.7521) (width 0.2) (layer "B.Cu") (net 4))
 (segment (start 87.0017 145.7521) (end 92.3028 151.0532) (width 0.2) (layer "B.Cu") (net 4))
 (segment (start 92.3028 151.0532) (end 93.452 152.2024) (width 0.2) (layer "B.Cu") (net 4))
 (segment (start 93.452 152.2024) (end 92.3028 151.0532) (width 0.2) (layer "B.Cu") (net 4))
 (segment (start 86 144.88) (end 87.0017 144.88) (width 0.2) (layer "B.Cu") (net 4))
 (segment (start 96.5 154.5) (end 97.2335 154.5) (width 0.2) (layer "F.Cu") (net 26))
 (segment (start 77.5 166) (end 78.4959 166.9959) (width 0.2) (layer "F.Cu") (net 26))
 (segment (start 80.5 166.3727) (end 80.5 152.3674) (width 0.2) (layer "F.Cu") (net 26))
 (segment (start 97.443 154.4644) (end 97.2691 154.4644) (width 0.2) (layer "F.Cu") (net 26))
 (segment (start 84.8726 151.8522) (end 84.8726 154.5005) (width 0.2) (layer "F.Cu") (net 26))
 (segment (start 83.94 150.9196) (end 84.8726 151.8522) (width 0.2) (layer "F.Cu") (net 26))
 (segment (start 80.5 152.3674) (end 81.9478 150.9196) (width 0.2) (layer "F.Cu") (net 26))
 (segment (start 82.51 138.505) (end 83.94 139.935) (width 0.2) (layer "F.Cu") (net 26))
 (segment (start 79.8768 166.9959) (end 80.5 166.3727) (width 0.2) (layer "F.Cu") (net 26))
 (segment (start 97.2691 154.4644) (end 97.2335 154.5) (width 0.2) (layer "F.Cu") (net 26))
 (segment (start 78.4959 166.9959) (end 79.8768 166.9959) (width 0.2) (layer "F.Cu") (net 26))
 (segment (start 83.94 139.935) (end 83.94 150.9196) (width 0.2) (layer "F.Cu") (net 26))
 (segment (start 81.9478 150.9196) (end 83.94 150.9196) (width 0.2) (layer "F.Cu") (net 26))
 (via (at 97.443 154.4644) (size 0.6) (drill 0.3) (layers "F.Cu" "B.Cu") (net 26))
 (via (at 84.8726 154.5005) (size 0.6) (drill 0.3) (layers "F.Cu" "B.Cu") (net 26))
 (segment (start 97.4069 154.5005) (end 97.443 154.4644) (width 0.2) (layer "B.Cu") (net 26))
 (segment (start 84.8726 154.5005) (end 97.4069 154.5005) (width 0.2) (layer "B.Cu") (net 26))
 (segment (start 91.68 148.5) (end 89.9683 148.5) (width 0.2) (layer "F.Cu") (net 5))
 (segment (start 91.5 150.9825) (end 91.5 166) (width 0.2) (layer "F.Cu") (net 5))
 (segment (start 89.9683 148.5) (end 89.9683 149.4508) (width 0.2) (layer "F.Cu") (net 5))
 (segment (start 89.9683 149.4508) (end 91.5 150.9825) (width 0.2) (layer "F.Cu") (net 5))
 (segment (start 91.5 166) (end 93.5 166) (width 0.2) (layer "B.Cu") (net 5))
 (segment (start 89.5 166) (end 91.5 166) (width 0.2) (layer "B.Cu") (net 5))
 (segment (start 75.5 135.63) (end 70.25 140.88) (width 1) (layer "F.Cu") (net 25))
 (segment (start 75.5 132) (end 75.5 135.63) (width 1) (layer "F.Cu") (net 25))
 (segment (start 71.7074 164.8369) (end 71.7074 151.4574) (width 1) (layer "F.Cu") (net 25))
 (segment (start 71.7074 151.4574) (end 70.25 150) (width 1) (layer "F.Cu") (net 25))
 (segment (start 71.5 165.0443) (end 71.7074 164.8369) (width 1) (layer "F.Cu") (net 25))
 (segment (start 70.25 150) (end 70.25 140.88) (width 1) (layer "F.Cu") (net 25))
 (segment (start 71.5 166) (end 71.5 165.0443) (width 1) (layer "F.Cu") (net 25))
 (segment (start 72.4557 166.3584) (end 73.0952 166.9979) (width 1) (layer "B.Cu") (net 25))
 (segment (start 73.0952 166.9979) (end 74.5021 166.9979) (width 1) (layer "B.Cu") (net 25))
 (segment (start 74.5021 166.9979) (end 75.5 166) (width 1) (layer "B.Cu") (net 25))
 (segment (start 71.5 166) (end 72.4557 166) (width 1) (layer "B.Cu") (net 25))
 (segment (start 72.4557 166) (end 72.4557 166.3584) (width 1) (layer "B.Cu") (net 25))
 (segment (start 83.5 162.485) (end 83.5 166) (width 1) (layer "F.Cu") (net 24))
 (segment (start 82.51 161.495) (end 83.5 162.485) (width 1) (layer "F.Cu") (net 24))
 (segment (start 68.199 128.611) (end 68.199 157.069) (width 1) (layer "F.Cu") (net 22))
 (segment (start 68.199 157.069) (end 70.25 159.12) (width 1) (layer "F.Cu") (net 22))
 (segment (start 68.199 123.611) (end 68.199 128.611) (width 1) (layer "F.Cu") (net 22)))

